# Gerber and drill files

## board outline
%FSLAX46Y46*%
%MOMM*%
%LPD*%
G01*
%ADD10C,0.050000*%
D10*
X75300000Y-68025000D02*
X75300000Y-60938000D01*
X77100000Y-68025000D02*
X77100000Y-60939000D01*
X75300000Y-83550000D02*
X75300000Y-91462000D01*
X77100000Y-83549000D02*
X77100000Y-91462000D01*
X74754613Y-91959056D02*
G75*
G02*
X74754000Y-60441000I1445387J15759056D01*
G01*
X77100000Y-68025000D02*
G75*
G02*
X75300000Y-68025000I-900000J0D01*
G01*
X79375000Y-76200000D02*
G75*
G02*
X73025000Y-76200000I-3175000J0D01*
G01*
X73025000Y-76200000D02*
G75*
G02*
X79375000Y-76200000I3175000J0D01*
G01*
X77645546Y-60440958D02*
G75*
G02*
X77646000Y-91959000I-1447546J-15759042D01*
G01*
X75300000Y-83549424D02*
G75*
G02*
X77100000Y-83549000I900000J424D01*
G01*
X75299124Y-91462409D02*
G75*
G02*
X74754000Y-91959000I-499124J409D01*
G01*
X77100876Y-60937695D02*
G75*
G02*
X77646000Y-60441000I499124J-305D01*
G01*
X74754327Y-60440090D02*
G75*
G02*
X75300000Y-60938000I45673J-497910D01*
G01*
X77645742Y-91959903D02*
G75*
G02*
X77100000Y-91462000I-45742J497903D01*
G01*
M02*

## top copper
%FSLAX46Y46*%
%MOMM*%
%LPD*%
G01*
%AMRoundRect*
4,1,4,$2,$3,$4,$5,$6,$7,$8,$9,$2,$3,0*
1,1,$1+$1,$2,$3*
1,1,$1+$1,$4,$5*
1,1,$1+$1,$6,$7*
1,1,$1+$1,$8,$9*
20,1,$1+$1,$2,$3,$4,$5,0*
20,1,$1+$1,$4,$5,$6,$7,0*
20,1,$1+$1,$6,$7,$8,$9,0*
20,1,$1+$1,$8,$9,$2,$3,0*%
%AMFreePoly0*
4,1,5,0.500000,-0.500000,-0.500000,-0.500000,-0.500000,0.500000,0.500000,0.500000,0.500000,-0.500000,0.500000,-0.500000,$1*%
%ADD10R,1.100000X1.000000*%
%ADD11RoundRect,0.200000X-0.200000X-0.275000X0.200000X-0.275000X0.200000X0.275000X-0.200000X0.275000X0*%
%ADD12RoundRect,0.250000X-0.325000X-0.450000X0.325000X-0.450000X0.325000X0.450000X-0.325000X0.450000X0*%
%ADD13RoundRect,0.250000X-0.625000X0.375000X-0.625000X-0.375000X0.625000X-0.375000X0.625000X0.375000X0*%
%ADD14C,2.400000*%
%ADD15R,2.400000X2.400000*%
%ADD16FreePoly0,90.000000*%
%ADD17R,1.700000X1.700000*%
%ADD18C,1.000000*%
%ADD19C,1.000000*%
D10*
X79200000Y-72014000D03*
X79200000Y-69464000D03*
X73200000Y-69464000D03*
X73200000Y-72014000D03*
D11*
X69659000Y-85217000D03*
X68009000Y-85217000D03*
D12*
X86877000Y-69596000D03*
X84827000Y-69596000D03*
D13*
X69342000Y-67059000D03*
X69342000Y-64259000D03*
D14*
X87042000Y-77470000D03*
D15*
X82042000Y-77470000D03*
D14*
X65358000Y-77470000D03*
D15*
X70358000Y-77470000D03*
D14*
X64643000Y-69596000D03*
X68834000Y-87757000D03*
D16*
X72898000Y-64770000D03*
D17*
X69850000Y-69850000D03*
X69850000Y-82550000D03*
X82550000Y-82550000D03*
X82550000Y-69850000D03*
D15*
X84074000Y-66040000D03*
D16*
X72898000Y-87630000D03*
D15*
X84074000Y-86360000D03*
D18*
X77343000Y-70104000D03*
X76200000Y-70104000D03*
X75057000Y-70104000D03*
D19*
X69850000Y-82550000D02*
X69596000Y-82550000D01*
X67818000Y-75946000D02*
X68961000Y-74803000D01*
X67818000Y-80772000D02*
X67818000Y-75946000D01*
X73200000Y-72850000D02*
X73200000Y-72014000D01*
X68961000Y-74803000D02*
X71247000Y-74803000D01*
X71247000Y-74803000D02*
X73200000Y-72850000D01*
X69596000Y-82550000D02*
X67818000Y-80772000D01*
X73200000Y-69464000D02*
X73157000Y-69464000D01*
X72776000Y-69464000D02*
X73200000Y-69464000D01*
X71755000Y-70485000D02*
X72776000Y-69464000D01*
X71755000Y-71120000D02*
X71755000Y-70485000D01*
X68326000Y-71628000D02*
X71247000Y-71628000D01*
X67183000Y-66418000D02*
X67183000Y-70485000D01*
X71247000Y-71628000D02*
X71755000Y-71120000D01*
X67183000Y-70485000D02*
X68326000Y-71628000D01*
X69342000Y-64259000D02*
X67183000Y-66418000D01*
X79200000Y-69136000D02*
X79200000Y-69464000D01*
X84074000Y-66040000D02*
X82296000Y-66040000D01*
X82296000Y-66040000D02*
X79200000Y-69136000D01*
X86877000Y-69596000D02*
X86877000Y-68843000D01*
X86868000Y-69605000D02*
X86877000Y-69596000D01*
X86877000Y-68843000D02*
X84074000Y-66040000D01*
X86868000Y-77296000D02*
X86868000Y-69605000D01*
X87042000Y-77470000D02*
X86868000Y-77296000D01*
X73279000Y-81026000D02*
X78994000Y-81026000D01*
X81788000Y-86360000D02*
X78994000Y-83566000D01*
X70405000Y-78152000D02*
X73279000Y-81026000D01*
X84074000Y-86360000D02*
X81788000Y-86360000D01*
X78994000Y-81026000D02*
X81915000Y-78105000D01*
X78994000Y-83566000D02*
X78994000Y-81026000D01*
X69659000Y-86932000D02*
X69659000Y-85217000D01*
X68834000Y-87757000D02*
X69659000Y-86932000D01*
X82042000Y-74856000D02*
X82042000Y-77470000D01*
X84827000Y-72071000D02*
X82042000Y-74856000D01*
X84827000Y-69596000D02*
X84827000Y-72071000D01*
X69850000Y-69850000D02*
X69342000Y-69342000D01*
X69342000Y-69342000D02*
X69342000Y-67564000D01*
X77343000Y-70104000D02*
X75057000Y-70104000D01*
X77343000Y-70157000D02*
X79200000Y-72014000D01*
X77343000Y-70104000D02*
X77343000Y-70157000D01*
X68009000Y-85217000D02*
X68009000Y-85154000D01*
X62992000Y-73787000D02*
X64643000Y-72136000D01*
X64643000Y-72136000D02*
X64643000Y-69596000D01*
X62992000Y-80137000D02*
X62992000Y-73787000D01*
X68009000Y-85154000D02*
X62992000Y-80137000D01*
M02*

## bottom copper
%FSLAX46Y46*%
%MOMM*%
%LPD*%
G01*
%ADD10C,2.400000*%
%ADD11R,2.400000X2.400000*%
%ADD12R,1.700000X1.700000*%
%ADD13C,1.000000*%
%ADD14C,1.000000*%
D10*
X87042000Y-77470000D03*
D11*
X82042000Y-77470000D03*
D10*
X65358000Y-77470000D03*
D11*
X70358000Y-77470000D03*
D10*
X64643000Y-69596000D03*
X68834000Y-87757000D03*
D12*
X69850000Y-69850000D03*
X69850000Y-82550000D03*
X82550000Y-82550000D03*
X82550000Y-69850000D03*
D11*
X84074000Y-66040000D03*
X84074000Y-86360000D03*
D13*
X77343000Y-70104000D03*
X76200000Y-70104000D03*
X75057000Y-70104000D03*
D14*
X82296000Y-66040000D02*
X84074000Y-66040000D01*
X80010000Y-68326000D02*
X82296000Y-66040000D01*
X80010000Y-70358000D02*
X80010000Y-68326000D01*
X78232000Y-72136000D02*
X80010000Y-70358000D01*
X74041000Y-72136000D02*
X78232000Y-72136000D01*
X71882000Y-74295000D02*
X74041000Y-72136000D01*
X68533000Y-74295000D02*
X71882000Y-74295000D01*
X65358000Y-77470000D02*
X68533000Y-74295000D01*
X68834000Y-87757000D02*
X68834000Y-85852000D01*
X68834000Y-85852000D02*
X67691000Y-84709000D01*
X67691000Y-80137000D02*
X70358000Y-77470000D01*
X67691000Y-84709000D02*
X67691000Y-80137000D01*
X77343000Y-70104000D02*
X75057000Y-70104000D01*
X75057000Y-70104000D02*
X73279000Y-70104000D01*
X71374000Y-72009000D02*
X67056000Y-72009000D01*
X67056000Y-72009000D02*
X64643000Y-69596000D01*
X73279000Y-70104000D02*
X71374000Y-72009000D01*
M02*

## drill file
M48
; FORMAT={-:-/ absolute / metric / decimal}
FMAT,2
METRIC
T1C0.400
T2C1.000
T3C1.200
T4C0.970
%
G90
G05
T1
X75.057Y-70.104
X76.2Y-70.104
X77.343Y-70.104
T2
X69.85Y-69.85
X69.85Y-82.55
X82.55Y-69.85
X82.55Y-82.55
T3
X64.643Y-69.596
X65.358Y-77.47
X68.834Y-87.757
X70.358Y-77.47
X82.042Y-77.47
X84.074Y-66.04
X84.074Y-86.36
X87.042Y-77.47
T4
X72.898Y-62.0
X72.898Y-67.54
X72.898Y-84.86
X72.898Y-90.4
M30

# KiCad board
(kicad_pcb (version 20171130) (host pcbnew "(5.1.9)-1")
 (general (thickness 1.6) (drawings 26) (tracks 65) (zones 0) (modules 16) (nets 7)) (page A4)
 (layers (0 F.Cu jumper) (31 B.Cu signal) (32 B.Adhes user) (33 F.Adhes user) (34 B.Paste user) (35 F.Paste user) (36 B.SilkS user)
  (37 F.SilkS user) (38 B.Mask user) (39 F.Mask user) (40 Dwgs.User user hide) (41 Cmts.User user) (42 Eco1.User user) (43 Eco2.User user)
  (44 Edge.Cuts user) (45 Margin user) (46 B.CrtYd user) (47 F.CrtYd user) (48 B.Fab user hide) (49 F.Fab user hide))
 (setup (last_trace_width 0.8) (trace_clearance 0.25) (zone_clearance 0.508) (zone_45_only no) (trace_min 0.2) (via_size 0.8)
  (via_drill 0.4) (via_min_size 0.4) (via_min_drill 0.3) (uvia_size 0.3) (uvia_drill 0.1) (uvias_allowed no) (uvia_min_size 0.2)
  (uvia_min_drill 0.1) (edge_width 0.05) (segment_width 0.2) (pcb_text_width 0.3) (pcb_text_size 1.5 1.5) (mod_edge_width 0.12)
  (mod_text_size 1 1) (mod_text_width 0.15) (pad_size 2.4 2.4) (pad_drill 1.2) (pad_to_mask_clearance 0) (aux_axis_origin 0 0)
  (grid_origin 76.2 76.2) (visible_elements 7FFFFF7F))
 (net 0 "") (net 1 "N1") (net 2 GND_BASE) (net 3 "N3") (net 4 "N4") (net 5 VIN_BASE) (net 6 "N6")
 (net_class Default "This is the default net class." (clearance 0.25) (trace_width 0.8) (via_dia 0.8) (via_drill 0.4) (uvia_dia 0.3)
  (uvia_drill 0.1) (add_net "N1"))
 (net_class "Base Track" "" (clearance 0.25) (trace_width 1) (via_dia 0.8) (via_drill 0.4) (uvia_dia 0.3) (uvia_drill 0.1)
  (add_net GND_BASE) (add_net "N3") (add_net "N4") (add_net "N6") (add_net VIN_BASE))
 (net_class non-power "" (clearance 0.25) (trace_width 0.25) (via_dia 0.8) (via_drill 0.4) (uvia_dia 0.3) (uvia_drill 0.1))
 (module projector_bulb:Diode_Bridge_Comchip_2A (layer F.Cu) (at 76.2 70.739 180)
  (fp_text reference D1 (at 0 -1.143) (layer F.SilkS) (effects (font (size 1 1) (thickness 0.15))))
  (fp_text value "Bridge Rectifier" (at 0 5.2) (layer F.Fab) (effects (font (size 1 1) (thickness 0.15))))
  (pad 1 smd rect (at -3 -1.275 180) (size 1.1 1) (layers F.Cu F.Paste F.Mask) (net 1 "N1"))
  (pad 2 smd rect (at -3 1.275 180) (size 1.1 1) (layers F.Cu F.Paste F.Mask) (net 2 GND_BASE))
  (pad 3 smd rect (at 3 1.275 180) (size 1.1 1) (layers F.Cu F.Paste F.Mask) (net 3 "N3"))
  (pad 4 smd rect (at 3 -1.275 180) (size 1.1 1) (layers F.Cu F.Paste F.Mask) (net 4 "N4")))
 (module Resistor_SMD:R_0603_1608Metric (layer F.Cu) (at 68.834 85.217)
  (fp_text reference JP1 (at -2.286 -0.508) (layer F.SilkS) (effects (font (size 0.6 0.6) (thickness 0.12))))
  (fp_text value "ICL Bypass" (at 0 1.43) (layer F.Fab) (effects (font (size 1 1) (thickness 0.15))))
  (pad 2 smd roundrect (at 0.825 0) (size 0.8 0.95) (layers F.Cu F.Paste F.Mask) (roundrect_rratio 0.25) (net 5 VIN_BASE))
  (pad 1 smd roundrect (at -0.825 0) (size 0.8 0.95) (layers F.Cu F.Paste F.Mask) (roundrect_rratio 0.25) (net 1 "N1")))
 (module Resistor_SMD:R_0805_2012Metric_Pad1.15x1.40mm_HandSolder (layer F.Cu) (at 85.852 69.596)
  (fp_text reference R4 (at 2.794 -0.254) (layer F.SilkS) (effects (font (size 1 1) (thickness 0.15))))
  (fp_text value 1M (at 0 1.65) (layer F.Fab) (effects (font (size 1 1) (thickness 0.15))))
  (pad 2 smd roundrect (at 1.025 0) (size 1.15 1.4) (layers F.Cu F.Paste F.Mask) (roundrect_rratio 0.217391) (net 2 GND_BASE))
  (pad 1 smd roundrect (at -1.025 0) (size 1.15 1.4) (layers F.Cu F.Paste F.Mask) (roundrect_rratio 0.217391) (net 5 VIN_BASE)))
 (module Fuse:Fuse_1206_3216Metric (layer F.Cu) (at 69.342 65.659 270)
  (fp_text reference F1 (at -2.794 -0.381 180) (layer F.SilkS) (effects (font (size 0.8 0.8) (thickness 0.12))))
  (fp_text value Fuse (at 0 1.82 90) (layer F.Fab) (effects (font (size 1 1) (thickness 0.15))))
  (pad 2 smd roundrect (at 1.4 0 270) (size 1.25 1.75) (layers F.Cu F.Paste F.Mask) (roundrect_rratio 0.2) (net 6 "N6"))
  (pad 1 smd roundrect (at -1.4 0 270) (size 1.25 1.75) (layers F.Cu F.Paste F.Mask) (roundrect_rratio 0.2) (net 3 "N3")))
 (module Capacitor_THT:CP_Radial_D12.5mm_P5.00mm (layer F.Cu) (at 82.042 77.47)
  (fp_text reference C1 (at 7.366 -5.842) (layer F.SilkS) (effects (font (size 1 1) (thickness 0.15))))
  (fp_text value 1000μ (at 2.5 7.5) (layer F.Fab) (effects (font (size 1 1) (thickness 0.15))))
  (pad 2 thru_hole circle (at 5 0) (size 2.4 2.4) (drill 1.2) (layers *.Cu *.Mask) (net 2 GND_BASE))
  (pad 1 thru_hole rect (at 0 0) (size 2.4 2.4) (drill 1.2) (layers *.Cu *.Mask) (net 5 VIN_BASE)))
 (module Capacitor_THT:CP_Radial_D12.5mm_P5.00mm (layer F.Cu) (at 70.358 77.47 180)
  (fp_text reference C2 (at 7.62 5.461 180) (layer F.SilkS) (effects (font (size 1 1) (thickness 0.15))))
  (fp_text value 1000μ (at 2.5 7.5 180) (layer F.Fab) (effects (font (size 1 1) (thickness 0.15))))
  (pad 2 thru_hole circle (at 5 0 180) (size 2.4 2.4) (drill 1.2) (layers *.Cu *.Mask) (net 2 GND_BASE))
  (pad 1 thru_hole rect (at 0 0 180) (size 2.4 2.4) (drill 1.2) (layers *.Cu *.Mask) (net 5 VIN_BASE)))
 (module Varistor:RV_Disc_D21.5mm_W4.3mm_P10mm (layer F.Cu) (at 64.897 82.042 90)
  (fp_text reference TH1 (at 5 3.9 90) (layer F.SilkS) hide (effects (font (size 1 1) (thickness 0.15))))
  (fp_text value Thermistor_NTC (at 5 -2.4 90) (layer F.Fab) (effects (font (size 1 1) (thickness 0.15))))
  (pad 2 thru_hole circle (at 12.446 -0.254 90) (size 2.4 2.4) (drill 1.2) (layers *.Cu *.Mask) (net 1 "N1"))
  (pad 1 thru_hole circle (at -5.715 3.937 90) (size 2.4 2.4) (drill 1.2) (layers *.Cu *.Mask) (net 5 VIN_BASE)))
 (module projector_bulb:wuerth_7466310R (layer F.Cu) (at 72.898 64.77 90)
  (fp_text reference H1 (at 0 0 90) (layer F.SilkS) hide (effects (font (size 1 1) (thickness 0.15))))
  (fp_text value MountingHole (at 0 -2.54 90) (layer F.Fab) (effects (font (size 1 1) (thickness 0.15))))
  (pad "" np_thru_hole circle (at -2.77 0 270) (size 0.97 0.97) (drill 0.97) (layers *.Cu *.Mask) (zone_connect 0))
  (pad "" np_thru_hole circle (at 2.77 0 90) (size 0.97 0.97) (drill 0.97) (layers *.Cu *.Mask) (zone_connect 0))
  (pad 1 smd custom (at 0 0 90) (size 1 1) (layers F.Cu F.Paste F.Mask) (zone_connect 0) (options (clearance outline) (anchor rect))
   (primitives)))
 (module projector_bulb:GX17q (layer B.Cu) (at 76.2 76.2)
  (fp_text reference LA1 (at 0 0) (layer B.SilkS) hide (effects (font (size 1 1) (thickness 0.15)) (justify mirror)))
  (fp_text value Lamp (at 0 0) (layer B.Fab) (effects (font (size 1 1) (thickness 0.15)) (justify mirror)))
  (pad 2 thru_hole rect (at -6.35 -6.35 90) (size 1.7 1.7) (drill 1) (layers *.Cu *.Mask) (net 6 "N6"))
  (pad 1 thru_hole rect (at -6.35 6.35 180) (size 1.7 1.7) (drill 1) (layers *.Cu *.Mask) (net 4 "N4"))
  (pad "" thru_hole rect (at 6.35 6.35 270) (size 1.7 1.7) (drill 1) (layers *.Cu *.Mask))
  (pad "" thru_hole rect (at 6.35 -6.35) (size 1.7 1.7) (drill 1) (layers *.Cu *.Mask)))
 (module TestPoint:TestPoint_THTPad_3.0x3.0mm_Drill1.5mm (layer F.Cu) (at 84.074 66.04)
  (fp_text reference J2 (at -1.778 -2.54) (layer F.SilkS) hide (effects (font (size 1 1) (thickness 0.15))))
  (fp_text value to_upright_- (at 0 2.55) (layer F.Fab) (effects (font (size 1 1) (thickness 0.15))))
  (pad 1 thru_hole rect (at 0 0) (size 2.4 2.4) (drill 1.2) (layers *.Cu *.Mask) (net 2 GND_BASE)))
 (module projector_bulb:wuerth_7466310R (layer F.Cu) (at 72.898 87.63 90)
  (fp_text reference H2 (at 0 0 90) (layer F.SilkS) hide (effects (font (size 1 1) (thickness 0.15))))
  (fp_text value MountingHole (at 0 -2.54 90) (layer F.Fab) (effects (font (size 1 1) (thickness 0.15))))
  (pad "" np_thru_hole circle (at -2.77 0 270) (size 0.97 0.97) (drill 0.97) (layers *.Cu *.Mask) (zone_connect 0))
  (pad "" np_thru_hole circle (at 2.77 0 90) (size 0.97 0.97) (drill 0.97) (layers *.Cu *.Mask) (zone_connect 0))
  (pad 1 smd custom (at 0 0 90) (size 1 1) (layers F.Cu F.Paste F.Mask) (zone_connect 0) (options (clearance outline) (anchor rect))
   (primitives)))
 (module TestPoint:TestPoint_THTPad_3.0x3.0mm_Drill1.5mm (layer F.Cu) (at 84.074 86.36)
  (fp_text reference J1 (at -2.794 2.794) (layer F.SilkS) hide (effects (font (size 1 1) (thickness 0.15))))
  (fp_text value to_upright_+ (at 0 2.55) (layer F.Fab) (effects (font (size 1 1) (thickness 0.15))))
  (pad 1 thru_hole rect (at 0 0) (size 2.4 2.4) (drill 1.2) (layers *.Cu *.Mask) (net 5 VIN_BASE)))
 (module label (layer F.Cu) (at 81.026 65.405 90)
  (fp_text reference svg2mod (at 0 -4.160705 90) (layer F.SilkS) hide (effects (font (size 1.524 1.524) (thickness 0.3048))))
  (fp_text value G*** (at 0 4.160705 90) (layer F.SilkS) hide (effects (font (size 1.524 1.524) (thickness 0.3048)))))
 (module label (layer F.Cu) (at 65.532 85.852 270)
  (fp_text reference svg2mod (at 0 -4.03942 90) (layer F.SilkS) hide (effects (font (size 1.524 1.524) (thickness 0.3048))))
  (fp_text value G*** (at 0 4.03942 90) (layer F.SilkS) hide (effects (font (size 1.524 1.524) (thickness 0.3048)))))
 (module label (layer F.Cu) (at 80.645 87.63 90)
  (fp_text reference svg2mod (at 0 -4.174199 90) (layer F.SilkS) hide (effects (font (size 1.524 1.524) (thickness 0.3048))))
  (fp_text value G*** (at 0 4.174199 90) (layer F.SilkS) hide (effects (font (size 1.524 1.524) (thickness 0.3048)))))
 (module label (layer F.Cu) (at 66.675 65.151 180)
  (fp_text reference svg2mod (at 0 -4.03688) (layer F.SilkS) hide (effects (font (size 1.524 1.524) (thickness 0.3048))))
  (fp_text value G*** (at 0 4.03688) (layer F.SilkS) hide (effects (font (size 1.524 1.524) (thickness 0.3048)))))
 (gr_line (start 75.3 68.025) (end 75.3 60.938) (angle 90) (layer Edge.Cuts) (width 0.05))
 (gr_line (start 77.1 68.025) (end 77.1 60.939) (angle 90) (layer Edge.Cuts) (width 0.05))
 (gr_line (start 75.3 83.55) (end 75.3 91.462) (angle 90) (layer Edge.Cuts) (width 0.05))
 (gr_line (start 77.1 83.549) (end 77.1 91.462) (angle 90) (layer Edge.Cuts) (width 0.05))
 (gr_arc (start 76.2 76.2) (end 74.754 60.441) (angle -169.517) (layer Edge.Cuts) (width 0.05))
 (gr_arc (start 76.2 68.025) (end 75.3 68.025) (angle -180) (layer Edge.Cuts) (width 0.05))
 (gr_circle (center 76.2 76.2) (end 73.025 76.2) (layer Edge.Cuts) (width 0.05))
 (gr_arc (start 76.198 76.2) (end 77.646 91.959) (angle -169.502) (layer Edge.Cuts) (width 0.05))
 (gr_arc (start 76.2 83.549) (end 77.1 83.549) (angle -180.027) (layer Edge.Cuts) (width 0.05))
 (gr_arc (start 74.8 91.462) (end 74.754 91.959) (angle -95.241) (layer Edge.Cuts) (width 0.05))
 (gr_arc (start 77.6 60.938) (end 77.646 60.441) (angle -95.253) (layer Edge.Cuts) (width 0.05))
 (gr_arc (start 74.8 60.938) (end 75.3 60.938) (angle -95.241) (layer Edge.Cuts) (width 0.05))
 (gr_arc (start 77.6 91.462) (end 77.1 91.462) (angle -95.249) (layer Edge.Cuts) (width 0.05))
 (segment (start 69.85 82.55) (end 69.596 82.55) (width 1) (layer F.Cu) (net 4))
 (segment (start 67.818 75.946) (end 68.961 74.803) (width 1) (layer F.Cu) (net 4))
 (segment (start 67.818 80.772) (end 67.818 75.946) (width 1) (layer F.Cu) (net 4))
 (segment (start 73.2 72.85) (end 73.2 72.014) (width 1) (layer F.Cu) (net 4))
 (segment (start 68.961 74.803) (end 71.247 74.803) (width 1) (layer F.Cu) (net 4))
 (segment (start 71.247 74.803) (end 73.2 72.85) (width 1) (layer F.Cu) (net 4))
 (segment (start 69.596 82.55) (end 67.818 80.772) (width 1) (layer F.Cu) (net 4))
 (segment (start 73.2 69.464) (end 73.157 69.464) (width 1) (layer F.Cu) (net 3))
 (segment (start 72.776 69.464) (end 73.2 69.464) (width 1) (layer F.Cu) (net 3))
 (segment (start 71.755 70.485) (end 72.776 69.464) (width 1) (layer F.Cu) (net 3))
 (segment (start 71.755 71.12) (end 71.755 70.485) (width 1) (layer F.Cu) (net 3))
 (segment (start 68.326 71.628) (end 71.247 71.628) (width 1) (layer F.Cu) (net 3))
 (segment (start 67.183 66.418) (end 67.183 70.485) (width 1) (layer F.Cu) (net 3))
 (segment (start 71.247 71.628) (end 71.755 71.12) (width 1) (layer F.Cu) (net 3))
 (segment (start 67.183 70.485) (end 68.326 71.628) (width 1) (layer F.Cu) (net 3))
 (segment (start 69.342 64.259) (end 67.183 66.418) (width 1) (layer F.Cu) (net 3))
 (segment (start 79.2 69.136) (end 79.2 69.464) (width 1) (layer F.Cu) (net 2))
 (segment (start 84.074 66.04) (end 82.296 66.04) (width 1) (layer F.Cu) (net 2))
 (segment (start 82.296 66.04) (end 79.2 69.136) (width 1) (layer F.Cu) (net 2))
 (segment (start 82.296 66.04) (end 84.074 66.04) (width 1) (layer B.Cu) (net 2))
 (segment (start 80.01 68.326) (end 82.296 66.04) (width 1) (layer B.Cu) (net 2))
 (segment (start 80.01 70.358) (end 80.01 68.326) (width 1) (layer B.Cu) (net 2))
 (segment (start 78.232 72.136) (end 80.01 70.358) (width 1) (layer B.Cu) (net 2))
 (segment (start 74.041 72.136) (end 78.232 72.136) (width 1) (layer B.Cu) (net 2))
 (segment (start 71.882 74.295) (end 74.041 72.136) (width 1) (layer B.Cu) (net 2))
 (segment (start 68.533 74.295) (end 71.882 74.295) (width 1) (layer B.Cu) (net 2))
 (segment (start 65.358 77.47) (end 68.533 74.295) (width 1) (layer B.Cu) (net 2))
 (segment (start 86.877 69.596) (end 86.877 68.843) (width 1) (layer F.Cu) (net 2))
 (segment (start 86.868 69.605) (end 86.877 69.596) (width 1) (layer F.Cu) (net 2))
 (segment (start 86.877 68.843) (end 84.074 66.04) (width 1) (layer F.Cu) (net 2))
 (segment (start 86.868 77.296) (end 86.868 69.605) (width 1) (layer F.Cu) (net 2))
 (segment (start 87.042 77.47) (end 86.868 77.296) (width 1) (layer F.Cu) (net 2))
 (segment (start 73.279 81.026) (end 78.994 81.026) (width 1) (layer F.Cu) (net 5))
 (segment (start 81.788 86.36) (end 78.994 83.566) (width 1) (layer F.Cu) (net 5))
 (segment (start 70.405 78.152) (end 73.279 81.026) (width 1) (layer F.Cu) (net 5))
 (segment (start 84.074 86.36) (end 81.788 86.36) (width 1) (layer F.Cu) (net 5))
 (segment (start 78.994 81.026) (end 81.915 78.105) (width 1) (layer F.Cu) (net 5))
 (segment (start 78.994 83.566) (end 78.994 81.026) (width 1) (layer F.Cu) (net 5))
 (segment (start 69.659 86.932) (end 69.659 85.217) (width 1) (layer F.Cu) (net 5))
 (segment (start 68.834 87.757) (end 69.659 86.932) (width 1) (layer F.Cu) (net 5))
 (segment (start 68.834 87.757) (end 68.834 85.852) (width 1) (layer B.Cu) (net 5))
 (segment (start 68.834 85.852) (end 67.691 84.709) (width 1) (layer B.Cu) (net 5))
 (segment (start 67.691 80.137) (end 70.358 77.47) (width 1) (layer B.Cu) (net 5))
 (segment (start 67.691 84.709) (end 67.691 80.137) (width 1) (layer B.Cu) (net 5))
 (segment (start 82.042 74.856) (end 82.042 77.47) (width 1) (layer F.Cu) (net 5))
 (segment (start 84.827 72.071) (end 82.042 74.856) (width 1) (layer F.Cu) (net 5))
 (segment (start 84.827 69.596) (end 84.827 72.071) (width 1) (layer F.Cu) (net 5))
 (segment (start 69.85 69.85) (end 69.342 69.342) (width 1) (layer F.Cu) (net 6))
 (segment (start 69.342 69.342) (end 69.342 67.564) (width 1) (layer F.Cu) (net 6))
 (via (at 77.343 70.104) (size 1) (drill 0.4) (layers F.Cu B.Cu) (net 1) (status 1000000))
 (via (at 76.2 70.104) (size 1) (drill 0.4) (layers F.Cu B.Cu) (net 1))
 (via (at 75.057 70.104) (size 1) (drill 0.4) (layers F.Cu B.Cu) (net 1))
 (segment (start 77.343 70.104) (end 75.057 70.104) (width 1) (layer F.Cu) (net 1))
 (segment (start 77.343 70.104) (end 75.057 70.104) (width 1) (layer B.Cu) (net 1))
 (segment (start 77.343 70.157) (end 79.2 72.014) (width 1) (layer F.Cu) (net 1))
 (segment (start 77.343 70.104) (end 77.343 70.157) (width 1) (layer F.Cu) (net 1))
 (segment (start 75.057 70.104) (end 73.279 70.104) (width 1) (layer B.Cu) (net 1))
 (segment (start 71.374 72.009) (end 67.056 72.009) (width 1) (layer B.Cu) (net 1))
 (segment (start 67.056 72.009) (end 64.643 69.596) (width 1) (layer B.Cu) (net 1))
 (segment (start 73.279 70.104) (end 71.374 72.009) (width 1) (layer B.Cu) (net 1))
 (segment (start 68.009 85.217) (end 68.009 85.154) (width 1) (layer F.Cu) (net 1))
 (segment (start 62.992 73.787) (end 64.643 72.136) (width 1) (layer F.Cu) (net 1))
 (segment (start 64.643 72.136) (end 64.643 69.596) (width 1) (layer F.Cu) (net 1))
 (segment (start 62.992 80.137) (end 62.992 73.787) (width 1) (layer F.Cu) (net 1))
 (segment (start 68.009 85.154) (end 62.992 80.137) (width 1) (layer F.Cu) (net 1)))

